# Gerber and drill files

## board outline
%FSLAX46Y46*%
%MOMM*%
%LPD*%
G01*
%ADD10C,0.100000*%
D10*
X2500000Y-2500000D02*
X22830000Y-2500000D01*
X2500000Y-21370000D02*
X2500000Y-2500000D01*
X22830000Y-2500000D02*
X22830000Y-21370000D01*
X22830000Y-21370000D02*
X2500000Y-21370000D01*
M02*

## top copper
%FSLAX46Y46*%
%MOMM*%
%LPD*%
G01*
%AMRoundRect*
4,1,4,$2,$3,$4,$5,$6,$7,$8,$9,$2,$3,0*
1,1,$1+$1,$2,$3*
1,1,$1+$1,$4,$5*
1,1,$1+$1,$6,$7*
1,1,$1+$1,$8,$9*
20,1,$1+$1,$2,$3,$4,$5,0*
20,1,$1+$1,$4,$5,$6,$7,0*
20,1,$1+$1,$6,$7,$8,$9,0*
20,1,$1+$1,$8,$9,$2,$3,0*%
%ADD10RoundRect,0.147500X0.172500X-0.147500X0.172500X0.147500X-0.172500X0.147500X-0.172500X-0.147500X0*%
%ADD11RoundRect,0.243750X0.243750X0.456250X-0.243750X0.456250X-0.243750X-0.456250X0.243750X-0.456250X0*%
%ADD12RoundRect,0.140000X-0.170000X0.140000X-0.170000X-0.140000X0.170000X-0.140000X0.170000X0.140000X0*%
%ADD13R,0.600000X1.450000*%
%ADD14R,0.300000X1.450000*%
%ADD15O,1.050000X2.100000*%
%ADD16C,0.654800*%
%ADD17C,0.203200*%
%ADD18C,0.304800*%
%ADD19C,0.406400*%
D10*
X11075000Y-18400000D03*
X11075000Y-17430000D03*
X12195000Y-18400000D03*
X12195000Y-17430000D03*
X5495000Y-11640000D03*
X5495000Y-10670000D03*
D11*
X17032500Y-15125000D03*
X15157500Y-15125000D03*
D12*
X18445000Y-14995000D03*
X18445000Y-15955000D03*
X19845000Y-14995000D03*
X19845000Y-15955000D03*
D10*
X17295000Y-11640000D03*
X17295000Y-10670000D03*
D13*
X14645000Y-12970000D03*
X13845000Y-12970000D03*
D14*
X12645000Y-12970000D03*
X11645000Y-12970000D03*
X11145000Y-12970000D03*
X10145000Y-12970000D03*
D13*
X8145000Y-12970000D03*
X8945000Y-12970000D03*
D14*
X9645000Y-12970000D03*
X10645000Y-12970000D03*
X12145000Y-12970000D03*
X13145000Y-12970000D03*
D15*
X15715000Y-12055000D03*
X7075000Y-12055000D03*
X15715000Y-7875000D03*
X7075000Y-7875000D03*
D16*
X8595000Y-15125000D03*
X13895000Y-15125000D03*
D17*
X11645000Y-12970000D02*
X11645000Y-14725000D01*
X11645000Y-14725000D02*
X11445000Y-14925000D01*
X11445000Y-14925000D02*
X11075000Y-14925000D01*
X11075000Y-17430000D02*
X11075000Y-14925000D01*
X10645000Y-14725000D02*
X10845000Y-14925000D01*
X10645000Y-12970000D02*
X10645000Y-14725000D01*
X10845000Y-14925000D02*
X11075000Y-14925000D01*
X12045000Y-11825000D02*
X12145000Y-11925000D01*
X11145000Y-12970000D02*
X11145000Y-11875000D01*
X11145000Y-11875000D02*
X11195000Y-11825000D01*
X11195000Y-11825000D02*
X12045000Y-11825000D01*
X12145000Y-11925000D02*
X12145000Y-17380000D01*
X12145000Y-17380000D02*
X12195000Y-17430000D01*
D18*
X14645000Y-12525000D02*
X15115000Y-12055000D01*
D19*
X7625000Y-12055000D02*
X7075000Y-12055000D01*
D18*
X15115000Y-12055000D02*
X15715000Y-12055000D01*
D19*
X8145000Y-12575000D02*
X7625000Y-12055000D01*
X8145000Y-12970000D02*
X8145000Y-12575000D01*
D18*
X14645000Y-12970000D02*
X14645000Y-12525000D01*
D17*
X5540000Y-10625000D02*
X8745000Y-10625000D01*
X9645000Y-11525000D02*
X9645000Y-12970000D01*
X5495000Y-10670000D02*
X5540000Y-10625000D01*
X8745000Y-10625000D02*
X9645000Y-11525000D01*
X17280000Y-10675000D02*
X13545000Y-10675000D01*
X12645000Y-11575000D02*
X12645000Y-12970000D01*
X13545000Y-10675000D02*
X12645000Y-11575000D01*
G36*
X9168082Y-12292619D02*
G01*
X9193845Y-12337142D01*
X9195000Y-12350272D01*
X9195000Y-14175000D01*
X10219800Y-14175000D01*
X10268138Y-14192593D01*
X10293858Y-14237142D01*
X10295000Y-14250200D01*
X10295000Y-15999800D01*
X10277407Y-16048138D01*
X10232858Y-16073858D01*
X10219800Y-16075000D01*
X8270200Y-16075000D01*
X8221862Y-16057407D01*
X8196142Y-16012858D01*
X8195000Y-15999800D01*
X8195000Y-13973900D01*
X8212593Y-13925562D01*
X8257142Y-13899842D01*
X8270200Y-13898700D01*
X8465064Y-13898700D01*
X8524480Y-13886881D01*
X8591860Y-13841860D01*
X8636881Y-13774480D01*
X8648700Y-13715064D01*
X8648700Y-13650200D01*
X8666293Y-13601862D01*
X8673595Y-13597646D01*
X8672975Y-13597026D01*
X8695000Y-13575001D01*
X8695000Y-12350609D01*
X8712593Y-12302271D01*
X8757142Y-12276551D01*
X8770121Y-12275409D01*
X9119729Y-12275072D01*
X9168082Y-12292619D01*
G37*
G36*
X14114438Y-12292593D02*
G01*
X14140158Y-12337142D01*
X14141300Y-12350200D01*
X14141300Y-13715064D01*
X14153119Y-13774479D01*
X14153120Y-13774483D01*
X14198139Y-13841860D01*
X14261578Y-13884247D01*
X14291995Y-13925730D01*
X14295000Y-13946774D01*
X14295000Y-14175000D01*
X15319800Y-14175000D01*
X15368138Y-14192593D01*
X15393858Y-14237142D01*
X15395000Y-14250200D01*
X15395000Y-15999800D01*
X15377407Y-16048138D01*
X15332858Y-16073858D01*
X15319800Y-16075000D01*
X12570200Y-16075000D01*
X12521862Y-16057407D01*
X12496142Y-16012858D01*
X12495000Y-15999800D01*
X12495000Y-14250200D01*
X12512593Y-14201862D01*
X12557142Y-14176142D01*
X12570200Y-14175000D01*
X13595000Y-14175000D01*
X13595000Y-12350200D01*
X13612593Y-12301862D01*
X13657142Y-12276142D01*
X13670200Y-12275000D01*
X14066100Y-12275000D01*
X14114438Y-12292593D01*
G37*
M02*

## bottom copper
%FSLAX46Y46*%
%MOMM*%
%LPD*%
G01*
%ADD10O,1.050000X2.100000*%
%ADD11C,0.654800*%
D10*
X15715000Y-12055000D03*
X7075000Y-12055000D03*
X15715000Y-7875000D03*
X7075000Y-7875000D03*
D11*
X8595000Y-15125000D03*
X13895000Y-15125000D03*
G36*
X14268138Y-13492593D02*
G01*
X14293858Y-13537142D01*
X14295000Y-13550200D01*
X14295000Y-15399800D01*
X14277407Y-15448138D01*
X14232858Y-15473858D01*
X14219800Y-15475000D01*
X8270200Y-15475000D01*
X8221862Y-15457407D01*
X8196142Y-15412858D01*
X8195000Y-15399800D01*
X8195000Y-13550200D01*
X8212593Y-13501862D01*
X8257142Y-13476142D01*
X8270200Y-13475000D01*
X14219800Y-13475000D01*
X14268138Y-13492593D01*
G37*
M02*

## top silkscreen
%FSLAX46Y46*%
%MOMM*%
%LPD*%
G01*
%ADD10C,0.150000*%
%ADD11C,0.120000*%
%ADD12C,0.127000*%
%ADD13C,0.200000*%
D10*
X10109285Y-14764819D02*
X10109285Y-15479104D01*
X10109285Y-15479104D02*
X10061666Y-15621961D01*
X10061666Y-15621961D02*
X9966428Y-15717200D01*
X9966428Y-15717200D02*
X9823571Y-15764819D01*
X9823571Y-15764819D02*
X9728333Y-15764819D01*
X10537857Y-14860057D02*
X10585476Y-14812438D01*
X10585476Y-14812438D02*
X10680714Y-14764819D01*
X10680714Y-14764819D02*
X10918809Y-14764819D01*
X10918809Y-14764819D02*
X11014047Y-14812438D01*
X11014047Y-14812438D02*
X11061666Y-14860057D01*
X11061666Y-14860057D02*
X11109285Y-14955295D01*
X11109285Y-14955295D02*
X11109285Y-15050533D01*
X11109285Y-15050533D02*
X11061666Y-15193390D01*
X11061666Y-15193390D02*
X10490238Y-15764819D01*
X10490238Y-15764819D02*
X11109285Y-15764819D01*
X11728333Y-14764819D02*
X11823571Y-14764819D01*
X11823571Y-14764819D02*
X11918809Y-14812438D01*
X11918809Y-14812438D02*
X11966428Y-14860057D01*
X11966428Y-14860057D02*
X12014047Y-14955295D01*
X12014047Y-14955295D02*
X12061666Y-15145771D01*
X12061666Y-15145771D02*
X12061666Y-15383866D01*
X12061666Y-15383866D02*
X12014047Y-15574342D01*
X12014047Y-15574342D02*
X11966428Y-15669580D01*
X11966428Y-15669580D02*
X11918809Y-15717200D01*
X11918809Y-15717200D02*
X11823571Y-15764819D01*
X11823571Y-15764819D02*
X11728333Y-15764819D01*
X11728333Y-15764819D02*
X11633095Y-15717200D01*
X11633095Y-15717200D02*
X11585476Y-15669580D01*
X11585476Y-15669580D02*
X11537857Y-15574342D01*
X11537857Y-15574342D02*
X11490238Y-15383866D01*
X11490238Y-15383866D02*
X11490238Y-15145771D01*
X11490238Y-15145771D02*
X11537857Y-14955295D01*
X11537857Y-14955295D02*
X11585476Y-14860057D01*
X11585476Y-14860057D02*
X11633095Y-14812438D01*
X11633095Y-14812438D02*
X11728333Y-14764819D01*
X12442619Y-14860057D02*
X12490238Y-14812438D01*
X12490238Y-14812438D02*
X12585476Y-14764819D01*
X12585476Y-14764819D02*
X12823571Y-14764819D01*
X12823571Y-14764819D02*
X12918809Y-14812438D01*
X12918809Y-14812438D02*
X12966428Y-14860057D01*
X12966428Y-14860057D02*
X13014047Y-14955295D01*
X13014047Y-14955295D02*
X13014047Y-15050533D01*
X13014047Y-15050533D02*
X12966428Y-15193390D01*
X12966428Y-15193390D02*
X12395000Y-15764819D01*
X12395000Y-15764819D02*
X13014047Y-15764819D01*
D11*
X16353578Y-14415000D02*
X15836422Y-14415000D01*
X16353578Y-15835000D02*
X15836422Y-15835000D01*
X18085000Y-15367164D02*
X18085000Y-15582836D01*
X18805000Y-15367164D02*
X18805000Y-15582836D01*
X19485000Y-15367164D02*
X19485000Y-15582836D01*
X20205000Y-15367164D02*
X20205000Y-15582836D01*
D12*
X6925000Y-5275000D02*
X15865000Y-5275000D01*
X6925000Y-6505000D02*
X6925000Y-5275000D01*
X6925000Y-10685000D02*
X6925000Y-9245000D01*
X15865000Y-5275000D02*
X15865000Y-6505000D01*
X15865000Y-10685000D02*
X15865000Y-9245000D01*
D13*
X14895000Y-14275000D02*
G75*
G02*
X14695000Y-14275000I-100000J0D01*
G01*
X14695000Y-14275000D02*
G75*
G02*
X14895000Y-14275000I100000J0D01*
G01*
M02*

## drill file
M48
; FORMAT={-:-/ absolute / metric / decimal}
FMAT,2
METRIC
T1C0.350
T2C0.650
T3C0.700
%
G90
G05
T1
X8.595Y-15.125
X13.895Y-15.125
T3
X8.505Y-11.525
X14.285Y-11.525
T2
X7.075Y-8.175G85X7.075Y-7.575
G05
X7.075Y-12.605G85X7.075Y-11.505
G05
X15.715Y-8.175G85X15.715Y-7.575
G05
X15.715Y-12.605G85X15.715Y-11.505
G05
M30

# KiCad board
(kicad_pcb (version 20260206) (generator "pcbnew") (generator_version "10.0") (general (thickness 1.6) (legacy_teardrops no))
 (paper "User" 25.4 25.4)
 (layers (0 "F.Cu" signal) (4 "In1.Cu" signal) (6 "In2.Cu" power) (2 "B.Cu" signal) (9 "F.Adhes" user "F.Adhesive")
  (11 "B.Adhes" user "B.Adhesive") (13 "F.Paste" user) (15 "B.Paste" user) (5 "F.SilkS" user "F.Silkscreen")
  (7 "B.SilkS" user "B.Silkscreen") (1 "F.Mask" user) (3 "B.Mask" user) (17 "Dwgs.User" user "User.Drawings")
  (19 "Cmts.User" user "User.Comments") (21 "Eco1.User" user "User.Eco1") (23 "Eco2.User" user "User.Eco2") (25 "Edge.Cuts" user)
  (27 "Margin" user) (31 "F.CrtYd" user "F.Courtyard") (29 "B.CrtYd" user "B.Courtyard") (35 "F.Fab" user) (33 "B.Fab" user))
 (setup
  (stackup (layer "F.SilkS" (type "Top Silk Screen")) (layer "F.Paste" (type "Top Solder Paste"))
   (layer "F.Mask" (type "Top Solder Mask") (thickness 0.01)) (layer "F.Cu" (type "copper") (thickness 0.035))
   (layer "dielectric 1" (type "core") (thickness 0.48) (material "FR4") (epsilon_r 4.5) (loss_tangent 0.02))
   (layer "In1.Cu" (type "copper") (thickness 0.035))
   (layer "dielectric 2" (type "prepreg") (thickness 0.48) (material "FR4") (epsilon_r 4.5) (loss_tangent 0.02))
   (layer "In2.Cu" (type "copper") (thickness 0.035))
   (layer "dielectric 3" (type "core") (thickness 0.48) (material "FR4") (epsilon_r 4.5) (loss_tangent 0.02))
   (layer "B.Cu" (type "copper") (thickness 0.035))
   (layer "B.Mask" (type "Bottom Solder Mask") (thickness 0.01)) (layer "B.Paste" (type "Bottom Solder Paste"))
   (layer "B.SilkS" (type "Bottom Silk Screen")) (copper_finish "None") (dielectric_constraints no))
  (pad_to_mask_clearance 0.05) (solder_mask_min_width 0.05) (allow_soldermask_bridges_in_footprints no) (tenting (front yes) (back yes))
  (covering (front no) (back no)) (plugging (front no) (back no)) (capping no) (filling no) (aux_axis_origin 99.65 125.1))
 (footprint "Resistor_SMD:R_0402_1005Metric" (layer "F.Cu") (at 11.075 17.915 90)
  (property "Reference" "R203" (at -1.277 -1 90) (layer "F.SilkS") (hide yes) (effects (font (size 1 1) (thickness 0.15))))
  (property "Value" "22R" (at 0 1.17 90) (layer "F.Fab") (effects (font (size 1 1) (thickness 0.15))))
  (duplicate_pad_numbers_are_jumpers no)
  (pad "1" smd roundrect (at -0.485 0 90) (size 0.59 0.64) (layers "F.Cu" "F.Mask" "F.Paste") (roundrect_rratio 0.25) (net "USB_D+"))
  (pad "2" smd roundrect (at 0.485 0 90) (size 0.59 0.64) (layers "F.Cu" "F.Mask" "F.Paste") (roundrect_rratio 0.25) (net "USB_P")))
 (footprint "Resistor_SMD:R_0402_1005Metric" (layer "F.Cu") (at 12.195 17.915 90)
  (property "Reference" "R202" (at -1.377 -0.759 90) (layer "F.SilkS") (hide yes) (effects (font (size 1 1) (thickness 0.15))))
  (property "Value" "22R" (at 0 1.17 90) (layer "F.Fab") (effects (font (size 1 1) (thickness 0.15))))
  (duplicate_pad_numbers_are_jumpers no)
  (pad "1" smd roundrect (at -0.485 0 90) (size 0.59 0.64) (layers "F.Cu" "F.Mask" "F.Paste") (roundrect_rratio 0.25) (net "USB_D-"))
  (pad "2" smd roundrect (at 0.485 0 90) (size 0.59 0.64) (layers "F.Cu" "F.Mask" "F.Paste") (roundrect_rratio 0.25) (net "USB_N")))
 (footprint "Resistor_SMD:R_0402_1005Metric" (layer "F.Cu") (at 5.495 11.155 90)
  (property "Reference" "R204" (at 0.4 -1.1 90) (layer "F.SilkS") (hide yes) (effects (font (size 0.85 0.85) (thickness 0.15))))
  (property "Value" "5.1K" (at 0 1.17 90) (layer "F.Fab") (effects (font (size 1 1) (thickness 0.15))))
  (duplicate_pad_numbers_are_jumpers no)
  (pad "1" smd roundrect (at -0.485 0 90) (size 0.59 0.64) (layers "F.Cu" "F.Mask" "F.Paste") (roundrect_rratio 0.25) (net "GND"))
  (pad "2" smd roundrect (at 0.485 0 90) (size 0.59 0.64) (layers "F.Cu" "F.Mask" "F.Paste") (roundrect_rratio 0.25) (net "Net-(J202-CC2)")))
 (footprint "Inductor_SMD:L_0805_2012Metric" (layer "F.Cu") (at 16.095 15.125 180)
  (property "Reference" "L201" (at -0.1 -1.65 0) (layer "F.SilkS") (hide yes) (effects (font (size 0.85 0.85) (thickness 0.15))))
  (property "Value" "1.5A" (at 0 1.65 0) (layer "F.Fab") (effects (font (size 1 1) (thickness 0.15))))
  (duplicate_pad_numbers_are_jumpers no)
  (fp_line (start -0.258578 0.71) (end 0.258578 0.71) (stroke (width 0.12) (type solid)) (layer "F.SilkS"))
  (fp_line (start -0.258578 -0.71) (end 0.258578 -0.71) (stroke (width 0.12) (type solid)) (layer "F.SilkS"))
  (pad "1" smd roundrect (at -0.9375 0 180) (size 0.975 1.4) (layers "F.Cu" "F.Mask" "F.Paste") (roundrect_rratio 0.25) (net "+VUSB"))
  (pad "2" smd roundrect (at 0.9375 0 180) (size 0.975 1.4) (layers "F.Cu" "F.Mask" "F.Paste") (roundrect_rratio 0.25)
   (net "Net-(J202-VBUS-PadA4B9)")))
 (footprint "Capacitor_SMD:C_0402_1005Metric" (layer "F.Cu") (at 18.445 15.475 -90)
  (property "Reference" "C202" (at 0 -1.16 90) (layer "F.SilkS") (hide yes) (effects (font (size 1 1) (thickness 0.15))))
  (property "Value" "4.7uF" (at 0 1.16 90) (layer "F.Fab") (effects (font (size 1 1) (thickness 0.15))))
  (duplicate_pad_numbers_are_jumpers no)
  (fp_line (start -0.107836 0.36) (end 0.107836 0.36) (stroke (width 0.12) (type solid)) (layer "F.SilkS"))
  (fp_line (start -0.107836 -0.36) (end 0.107836 -0.36) (stroke (width 0.12) (type solid)) (layer "F.SilkS"))
  (pad "1" smd roundrect (at -0.48 0 270) (size 0.56 0.62) (layers "F.Cu" "F.Mask" "F.Paste") (roundrect_rratio 0.25) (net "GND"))
  (pad "2" smd roundrect (at 0.48 0 270) (size 0.56 0.62) (layers "F.Cu" "F.Mask" "F.Paste") (roundrect_rratio 0.25) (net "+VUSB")))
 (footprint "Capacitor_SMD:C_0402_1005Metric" (layer "F.Cu") (at 19.845 15.475 -90)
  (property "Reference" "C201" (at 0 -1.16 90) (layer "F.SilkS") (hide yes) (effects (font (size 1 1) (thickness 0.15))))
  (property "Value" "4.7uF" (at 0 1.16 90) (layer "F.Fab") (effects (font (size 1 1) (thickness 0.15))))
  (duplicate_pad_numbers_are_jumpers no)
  (fp_line (start -0.107836 0.36) (end 0.107836 0.36) (stroke (width 0.12) (type solid)) (layer "F.SilkS"))
  (fp_line (start -0.107836 -0.36) (end 0.107836 -0.36) (stroke (width 0.12) (type solid)) (layer "F.SilkS"))
  (pad "1" smd roundrect (at -0.48 0 270) (size 0.56 0.62) (layers "F.Cu" "F.Mask" "F.Paste") (roundrect_rratio 0.25) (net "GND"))
  (pad "2" smd roundrect (at 0.48 0 270) (size 0.56 0.62) (layers "F.Cu" "F.Mask" "F.Paste") (roundrect_rratio 0.25) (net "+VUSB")))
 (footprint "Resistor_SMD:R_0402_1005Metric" (layer "F.Cu") (at 17.295 11.155 90)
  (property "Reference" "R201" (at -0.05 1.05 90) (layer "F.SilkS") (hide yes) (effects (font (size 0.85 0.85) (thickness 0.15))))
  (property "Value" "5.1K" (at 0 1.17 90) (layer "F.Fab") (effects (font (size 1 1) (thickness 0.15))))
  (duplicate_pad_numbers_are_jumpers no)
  (pad "1" smd roundrect (at -0.485 0 90) (size 0.59 0.64) (layers "F.Cu" "F.Mask" "F.Paste") (roundrect_rratio 0.25) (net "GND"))
  (pad "2" smd roundrect (at 0.485 0 90) (size 0.59 0.64) (layers "F.Cu" "F.Mask" "F.Paste") (roundrect_rratio 0.25) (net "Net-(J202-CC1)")))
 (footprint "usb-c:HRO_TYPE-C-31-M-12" (layer "F.Cu") (at 11.395 7.875 180)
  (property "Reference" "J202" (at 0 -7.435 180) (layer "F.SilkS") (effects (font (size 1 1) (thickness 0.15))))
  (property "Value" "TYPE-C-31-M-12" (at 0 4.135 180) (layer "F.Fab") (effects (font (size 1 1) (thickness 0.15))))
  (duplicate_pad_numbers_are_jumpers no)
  (fp_line (start 4.47 2.6) (end -4.47 2.6) (stroke (width 0.127) (type solid)) (layer "F.SilkS"))
  (fp_line (start 4.47 1.37) (end 4.47 2.6) (stroke (width 0.127) (type solid)) (layer "F.SilkS"))
  (fp_line (start 4.47 -2.81) (end 4.47 -1.37) (stroke (width 0.127) (type solid)) (layer "F.SilkS"))
  (fp_line (start -4.47 2.6) (end -4.47 1.37) (stroke (width 0.127) (type solid)) (layer "F.SilkS"))
  (fp_line (start -4.47 -2.81) (end -4.47 -1.37) (stroke (width 0.127) (type solid)) (layer "F.SilkS"))
  (fp_circle (center -3.4 -6.4) (end -3.3 -6.4) (stroke (width 0.2) (type solid)) (fill no) (layer "F.SilkS"))
  (pad "" np_thru_hole circle (at -2.89 -3.65 180) (size 0.7 0.7) (drill 0.7) (layers "*.Cu" "*.Mask"))
  (pad "" np_thru_hole circle (at 2.89 -3.65 180) (size 0.7 0.7) (drill 0.7) (layers "*.Cu" "*.Mask"))
  (pad "A1B12" smd rect (at -3.25 -5.095 180) (size 0.6 1.45) (layers "F.Cu" "F.Mask" "F.Paste") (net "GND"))
  (pad "A4B9" smd rect (at -2.45 -5.095 180) (size 0.6 1.45) (layers "F.Cu" "F.Mask" "F.Paste") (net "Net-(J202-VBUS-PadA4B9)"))
  (pad "A5" smd rect (at -1.25 -5.095 180) (size 0.3 1.45) (layers "F.Cu" "F.Mask" "F.Paste") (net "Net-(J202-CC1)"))
  (pad "A6" smd rect (at -0.25 -5.095 180) (size 0.3 1.45) (layers "F.Cu" "F.Mask" "F.Paste") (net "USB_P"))
  (pad "A7" smd rect (at 0.25 -5.095 180) (size 0.3 1.45) (layers "F.Cu" "F.Mask" "F.Paste") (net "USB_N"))
  (pad "A8" smd rect (at 1.25 -5.095 180) (size 0.3 1.45) (layers "F.Cu" "F.Mask" "F.Paste") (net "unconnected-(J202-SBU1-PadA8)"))
  (pad "B1A12" smd rect (at 3.25 -5.095 180) (size 0.6 1.45) (layers "F.Cu" "F.Mask" "F.Paste") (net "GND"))
  (pad "B4A9" smd rect (at 2.45 -5.095 180) (size 0.6 1.45) (layers "F.Cu" "F.Mask" "F.Paste") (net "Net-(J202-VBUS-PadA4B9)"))
  (pad "B5" smd rect (at 1.75 -5.095 180) (size 0.3 1.45) (layers "F.Cu" "F.Mask" "F.Paste") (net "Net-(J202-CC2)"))
  (pad "B6" smd rect (at 0.75 -5.095 180) (size 0.3 1.45) (layers "F.Cu" "F.Mask" "F.Paste") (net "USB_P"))
  (pad "B7" smd rect (at -0.75 -5.095 180) (size 0.3 1.45) (layers "F.Cu" "F.Mask" "F.Paste") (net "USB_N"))
  (pad "B8" smd rect (at -1.75 -5.095 180) (size 0.3 1.45) (layers "F.Cu" "F.Mask" "F.Paste") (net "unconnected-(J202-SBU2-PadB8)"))
  (pad "S1" thru_hole oval (at -4.32 -4.18 180) (size 1.05 2.1) (drill oval 0.65 1.75) (layers "*.Cu" "*.Mask") (remove_unused_layers no)
   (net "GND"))
  (pad "S2" thru_hole oval (at 4.32 -4.18 180) (size 1.05 2.1) (drill oval 0.65 1.75) (layers "*.Cu" "*.Mask") (remove_unused_layers no)
   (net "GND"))
  (pad "S3" thru_hole oval (at -4.32 0 180) (size 1.05 2.1) (drill oval 0.65 1.25) (layers "*.Cu" "*.Mask") (remove_unused_layers no)
   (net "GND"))
  (pad "S4" thru_hole oval (at 4.32 0 180) (size 1.05 2.1) (drill oval 0.65 1.25) (layers "*.Cu" "*.Mask") (remove_unused_layers no)
   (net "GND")))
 (gr_line (start 2.5 2.5) (end 22.83 2.5) (stroke (width 0.1) (type default)) (layer "Edge.Cuts"))
 (gr_line (start 2.5 21.37) (end 2.5 2.5) (stroke (width 0.1) (type default)) (layer "Edge.Cuts"))
 (gr_line (start 22.83 2.5) (end 22.83 21.37) (stroke (width 0.1) (type default)) (layer "Edge.Cuts"))
 (gr_line (start 22.83 21.37) (end 2.5 21.37) (stroke (width 0.1) (type default)) (layer "Edge.Cuts"))
 (segment (start 11.645 12.97) (end 11.645 14.725) (width 0.2032) (layer "F.Cu") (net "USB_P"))
 (segment (start 11.645 14.725) (end 11.445 14.925) (width 0.2032) (layer "F.Cu") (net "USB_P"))
 (segment (start 11.445 14.925) (end 11.075 14.925) (width 0.2032) (layer "F.Cu") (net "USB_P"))
 (segment (start 11.075 17.43) (end 11.075 14.925) (width 0.2032) (layer "F.Cu") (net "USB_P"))
 (segment (start 10.645 14.725) (end 10.845 14.925) (width 0.2032) (layer "F.Cu") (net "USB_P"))
 (segment (start 10.645 12.97) (end 10.645 14.725) (width 0.2032) (layer "F.Cu") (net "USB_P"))
 (segment (start 10.845 14.925) (end 11.075 14.925) (width 0.2032) (layer "F.Cu") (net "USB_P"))
 (segment (start 12.045 11.825) (end 12.145 11.925) (width 0.2032) (layer "F.Cu") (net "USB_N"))
 (segment (start 11.145 12.97) (end 11.145 11.875) (width 0.2032) (layer "F.Cu") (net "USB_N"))
 (segment (start 11.145 11.875) (end 11.195 11.825) (width 0.2032) (layer "F.Cu") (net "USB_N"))
 (segment (start 11.195 11.825) (end 12.045 11.825) (width 0.2032) (layer "F.Cu") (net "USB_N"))
 (segment (start 12.145 11.925) (end 12.145 17.38) (width 0.2032) (layer "F.Cu") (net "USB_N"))
 (segment (start 12.145 17.38) (end 12.195 17.43) (width 0.2032) (layer "F.Cu") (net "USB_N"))
 (segment (start 14.645 12.525) (end 15.115 12.055) (width 0.3048) (layer "F.Cu") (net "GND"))
 (segment (start 7.625 12.055) (end 7.075 12.055) (width 0.4064) (layer "F.Cu") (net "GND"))
 (segment (start 15.115 12.055) (end 15.715 12.055) (width 0.3048) (layer "F.Cu") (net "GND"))
 (segment (start 8.145 12.575) (end 7.625 12.055) (width 0.4064) (layer "F.Cu") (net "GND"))
 (segment (start 8.145 12.97) (end 8.145 12.575) (width 0.4064) (layer "F.Cu") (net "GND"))
 (segment (start 14.645 12.97) (end 14.645 12.525) (width 0.3048) (layer "F.Cu") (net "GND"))
 (segment (start 5.54 10.625) (end 8.745 10.625) (width 0.2032) (layer "F.Cu") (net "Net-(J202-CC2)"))
 (segment (start 9.645 11.525) (end 9.645 12.97) (width 0.2032) (layer "F.Cu") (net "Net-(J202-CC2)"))
 (segment (start 5.495 10.67) (end 5.54 10.625) (width 0.2032) (layer "F.Cu") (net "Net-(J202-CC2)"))
 (segment (start 8.745 10.625) (end 9.645 11.525) (width 0.2032) (layer "F.Cu") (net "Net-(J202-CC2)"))
 (via (at 8.595 15.125) (size 0.6548) (drill 0.35) (layers "F.Cu" "B.Cu") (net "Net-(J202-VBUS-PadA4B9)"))
 (via (at 13.895 15.125) (size 0.6548) (drill 0.35) (layers "F.Cu" "B.Cu") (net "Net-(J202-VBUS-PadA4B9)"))
 (segment (start 17.28 10.675) (end 13.545 10.675) (width 0.2032) (layer "F.Cu") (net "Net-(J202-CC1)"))
 (segment (start 12.645 11.575) (end 12.645 12.97) (width 0.2032) (layer "F.Cu") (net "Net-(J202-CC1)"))
 (segment (start 13.545 10.675) (end 12.645 11.575) (width 0.2032) (layer "F.Cu") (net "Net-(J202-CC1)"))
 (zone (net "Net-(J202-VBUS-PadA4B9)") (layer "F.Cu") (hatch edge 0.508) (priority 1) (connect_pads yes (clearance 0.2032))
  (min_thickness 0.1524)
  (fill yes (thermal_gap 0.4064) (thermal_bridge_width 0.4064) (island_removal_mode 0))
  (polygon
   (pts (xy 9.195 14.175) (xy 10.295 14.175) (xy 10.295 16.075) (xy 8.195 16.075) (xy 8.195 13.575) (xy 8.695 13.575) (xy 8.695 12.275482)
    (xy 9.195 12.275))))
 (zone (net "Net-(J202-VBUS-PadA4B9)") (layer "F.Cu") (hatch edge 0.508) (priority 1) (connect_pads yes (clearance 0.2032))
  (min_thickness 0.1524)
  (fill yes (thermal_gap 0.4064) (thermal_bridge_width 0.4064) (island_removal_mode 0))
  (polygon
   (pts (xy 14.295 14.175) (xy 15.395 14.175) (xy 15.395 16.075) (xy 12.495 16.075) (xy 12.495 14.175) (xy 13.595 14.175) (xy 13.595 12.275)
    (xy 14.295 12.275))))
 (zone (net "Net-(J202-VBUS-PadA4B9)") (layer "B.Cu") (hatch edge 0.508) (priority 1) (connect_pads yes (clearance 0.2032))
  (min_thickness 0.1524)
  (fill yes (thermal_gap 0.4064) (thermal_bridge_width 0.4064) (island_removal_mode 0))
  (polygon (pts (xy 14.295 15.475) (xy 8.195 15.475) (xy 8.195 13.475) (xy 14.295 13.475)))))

